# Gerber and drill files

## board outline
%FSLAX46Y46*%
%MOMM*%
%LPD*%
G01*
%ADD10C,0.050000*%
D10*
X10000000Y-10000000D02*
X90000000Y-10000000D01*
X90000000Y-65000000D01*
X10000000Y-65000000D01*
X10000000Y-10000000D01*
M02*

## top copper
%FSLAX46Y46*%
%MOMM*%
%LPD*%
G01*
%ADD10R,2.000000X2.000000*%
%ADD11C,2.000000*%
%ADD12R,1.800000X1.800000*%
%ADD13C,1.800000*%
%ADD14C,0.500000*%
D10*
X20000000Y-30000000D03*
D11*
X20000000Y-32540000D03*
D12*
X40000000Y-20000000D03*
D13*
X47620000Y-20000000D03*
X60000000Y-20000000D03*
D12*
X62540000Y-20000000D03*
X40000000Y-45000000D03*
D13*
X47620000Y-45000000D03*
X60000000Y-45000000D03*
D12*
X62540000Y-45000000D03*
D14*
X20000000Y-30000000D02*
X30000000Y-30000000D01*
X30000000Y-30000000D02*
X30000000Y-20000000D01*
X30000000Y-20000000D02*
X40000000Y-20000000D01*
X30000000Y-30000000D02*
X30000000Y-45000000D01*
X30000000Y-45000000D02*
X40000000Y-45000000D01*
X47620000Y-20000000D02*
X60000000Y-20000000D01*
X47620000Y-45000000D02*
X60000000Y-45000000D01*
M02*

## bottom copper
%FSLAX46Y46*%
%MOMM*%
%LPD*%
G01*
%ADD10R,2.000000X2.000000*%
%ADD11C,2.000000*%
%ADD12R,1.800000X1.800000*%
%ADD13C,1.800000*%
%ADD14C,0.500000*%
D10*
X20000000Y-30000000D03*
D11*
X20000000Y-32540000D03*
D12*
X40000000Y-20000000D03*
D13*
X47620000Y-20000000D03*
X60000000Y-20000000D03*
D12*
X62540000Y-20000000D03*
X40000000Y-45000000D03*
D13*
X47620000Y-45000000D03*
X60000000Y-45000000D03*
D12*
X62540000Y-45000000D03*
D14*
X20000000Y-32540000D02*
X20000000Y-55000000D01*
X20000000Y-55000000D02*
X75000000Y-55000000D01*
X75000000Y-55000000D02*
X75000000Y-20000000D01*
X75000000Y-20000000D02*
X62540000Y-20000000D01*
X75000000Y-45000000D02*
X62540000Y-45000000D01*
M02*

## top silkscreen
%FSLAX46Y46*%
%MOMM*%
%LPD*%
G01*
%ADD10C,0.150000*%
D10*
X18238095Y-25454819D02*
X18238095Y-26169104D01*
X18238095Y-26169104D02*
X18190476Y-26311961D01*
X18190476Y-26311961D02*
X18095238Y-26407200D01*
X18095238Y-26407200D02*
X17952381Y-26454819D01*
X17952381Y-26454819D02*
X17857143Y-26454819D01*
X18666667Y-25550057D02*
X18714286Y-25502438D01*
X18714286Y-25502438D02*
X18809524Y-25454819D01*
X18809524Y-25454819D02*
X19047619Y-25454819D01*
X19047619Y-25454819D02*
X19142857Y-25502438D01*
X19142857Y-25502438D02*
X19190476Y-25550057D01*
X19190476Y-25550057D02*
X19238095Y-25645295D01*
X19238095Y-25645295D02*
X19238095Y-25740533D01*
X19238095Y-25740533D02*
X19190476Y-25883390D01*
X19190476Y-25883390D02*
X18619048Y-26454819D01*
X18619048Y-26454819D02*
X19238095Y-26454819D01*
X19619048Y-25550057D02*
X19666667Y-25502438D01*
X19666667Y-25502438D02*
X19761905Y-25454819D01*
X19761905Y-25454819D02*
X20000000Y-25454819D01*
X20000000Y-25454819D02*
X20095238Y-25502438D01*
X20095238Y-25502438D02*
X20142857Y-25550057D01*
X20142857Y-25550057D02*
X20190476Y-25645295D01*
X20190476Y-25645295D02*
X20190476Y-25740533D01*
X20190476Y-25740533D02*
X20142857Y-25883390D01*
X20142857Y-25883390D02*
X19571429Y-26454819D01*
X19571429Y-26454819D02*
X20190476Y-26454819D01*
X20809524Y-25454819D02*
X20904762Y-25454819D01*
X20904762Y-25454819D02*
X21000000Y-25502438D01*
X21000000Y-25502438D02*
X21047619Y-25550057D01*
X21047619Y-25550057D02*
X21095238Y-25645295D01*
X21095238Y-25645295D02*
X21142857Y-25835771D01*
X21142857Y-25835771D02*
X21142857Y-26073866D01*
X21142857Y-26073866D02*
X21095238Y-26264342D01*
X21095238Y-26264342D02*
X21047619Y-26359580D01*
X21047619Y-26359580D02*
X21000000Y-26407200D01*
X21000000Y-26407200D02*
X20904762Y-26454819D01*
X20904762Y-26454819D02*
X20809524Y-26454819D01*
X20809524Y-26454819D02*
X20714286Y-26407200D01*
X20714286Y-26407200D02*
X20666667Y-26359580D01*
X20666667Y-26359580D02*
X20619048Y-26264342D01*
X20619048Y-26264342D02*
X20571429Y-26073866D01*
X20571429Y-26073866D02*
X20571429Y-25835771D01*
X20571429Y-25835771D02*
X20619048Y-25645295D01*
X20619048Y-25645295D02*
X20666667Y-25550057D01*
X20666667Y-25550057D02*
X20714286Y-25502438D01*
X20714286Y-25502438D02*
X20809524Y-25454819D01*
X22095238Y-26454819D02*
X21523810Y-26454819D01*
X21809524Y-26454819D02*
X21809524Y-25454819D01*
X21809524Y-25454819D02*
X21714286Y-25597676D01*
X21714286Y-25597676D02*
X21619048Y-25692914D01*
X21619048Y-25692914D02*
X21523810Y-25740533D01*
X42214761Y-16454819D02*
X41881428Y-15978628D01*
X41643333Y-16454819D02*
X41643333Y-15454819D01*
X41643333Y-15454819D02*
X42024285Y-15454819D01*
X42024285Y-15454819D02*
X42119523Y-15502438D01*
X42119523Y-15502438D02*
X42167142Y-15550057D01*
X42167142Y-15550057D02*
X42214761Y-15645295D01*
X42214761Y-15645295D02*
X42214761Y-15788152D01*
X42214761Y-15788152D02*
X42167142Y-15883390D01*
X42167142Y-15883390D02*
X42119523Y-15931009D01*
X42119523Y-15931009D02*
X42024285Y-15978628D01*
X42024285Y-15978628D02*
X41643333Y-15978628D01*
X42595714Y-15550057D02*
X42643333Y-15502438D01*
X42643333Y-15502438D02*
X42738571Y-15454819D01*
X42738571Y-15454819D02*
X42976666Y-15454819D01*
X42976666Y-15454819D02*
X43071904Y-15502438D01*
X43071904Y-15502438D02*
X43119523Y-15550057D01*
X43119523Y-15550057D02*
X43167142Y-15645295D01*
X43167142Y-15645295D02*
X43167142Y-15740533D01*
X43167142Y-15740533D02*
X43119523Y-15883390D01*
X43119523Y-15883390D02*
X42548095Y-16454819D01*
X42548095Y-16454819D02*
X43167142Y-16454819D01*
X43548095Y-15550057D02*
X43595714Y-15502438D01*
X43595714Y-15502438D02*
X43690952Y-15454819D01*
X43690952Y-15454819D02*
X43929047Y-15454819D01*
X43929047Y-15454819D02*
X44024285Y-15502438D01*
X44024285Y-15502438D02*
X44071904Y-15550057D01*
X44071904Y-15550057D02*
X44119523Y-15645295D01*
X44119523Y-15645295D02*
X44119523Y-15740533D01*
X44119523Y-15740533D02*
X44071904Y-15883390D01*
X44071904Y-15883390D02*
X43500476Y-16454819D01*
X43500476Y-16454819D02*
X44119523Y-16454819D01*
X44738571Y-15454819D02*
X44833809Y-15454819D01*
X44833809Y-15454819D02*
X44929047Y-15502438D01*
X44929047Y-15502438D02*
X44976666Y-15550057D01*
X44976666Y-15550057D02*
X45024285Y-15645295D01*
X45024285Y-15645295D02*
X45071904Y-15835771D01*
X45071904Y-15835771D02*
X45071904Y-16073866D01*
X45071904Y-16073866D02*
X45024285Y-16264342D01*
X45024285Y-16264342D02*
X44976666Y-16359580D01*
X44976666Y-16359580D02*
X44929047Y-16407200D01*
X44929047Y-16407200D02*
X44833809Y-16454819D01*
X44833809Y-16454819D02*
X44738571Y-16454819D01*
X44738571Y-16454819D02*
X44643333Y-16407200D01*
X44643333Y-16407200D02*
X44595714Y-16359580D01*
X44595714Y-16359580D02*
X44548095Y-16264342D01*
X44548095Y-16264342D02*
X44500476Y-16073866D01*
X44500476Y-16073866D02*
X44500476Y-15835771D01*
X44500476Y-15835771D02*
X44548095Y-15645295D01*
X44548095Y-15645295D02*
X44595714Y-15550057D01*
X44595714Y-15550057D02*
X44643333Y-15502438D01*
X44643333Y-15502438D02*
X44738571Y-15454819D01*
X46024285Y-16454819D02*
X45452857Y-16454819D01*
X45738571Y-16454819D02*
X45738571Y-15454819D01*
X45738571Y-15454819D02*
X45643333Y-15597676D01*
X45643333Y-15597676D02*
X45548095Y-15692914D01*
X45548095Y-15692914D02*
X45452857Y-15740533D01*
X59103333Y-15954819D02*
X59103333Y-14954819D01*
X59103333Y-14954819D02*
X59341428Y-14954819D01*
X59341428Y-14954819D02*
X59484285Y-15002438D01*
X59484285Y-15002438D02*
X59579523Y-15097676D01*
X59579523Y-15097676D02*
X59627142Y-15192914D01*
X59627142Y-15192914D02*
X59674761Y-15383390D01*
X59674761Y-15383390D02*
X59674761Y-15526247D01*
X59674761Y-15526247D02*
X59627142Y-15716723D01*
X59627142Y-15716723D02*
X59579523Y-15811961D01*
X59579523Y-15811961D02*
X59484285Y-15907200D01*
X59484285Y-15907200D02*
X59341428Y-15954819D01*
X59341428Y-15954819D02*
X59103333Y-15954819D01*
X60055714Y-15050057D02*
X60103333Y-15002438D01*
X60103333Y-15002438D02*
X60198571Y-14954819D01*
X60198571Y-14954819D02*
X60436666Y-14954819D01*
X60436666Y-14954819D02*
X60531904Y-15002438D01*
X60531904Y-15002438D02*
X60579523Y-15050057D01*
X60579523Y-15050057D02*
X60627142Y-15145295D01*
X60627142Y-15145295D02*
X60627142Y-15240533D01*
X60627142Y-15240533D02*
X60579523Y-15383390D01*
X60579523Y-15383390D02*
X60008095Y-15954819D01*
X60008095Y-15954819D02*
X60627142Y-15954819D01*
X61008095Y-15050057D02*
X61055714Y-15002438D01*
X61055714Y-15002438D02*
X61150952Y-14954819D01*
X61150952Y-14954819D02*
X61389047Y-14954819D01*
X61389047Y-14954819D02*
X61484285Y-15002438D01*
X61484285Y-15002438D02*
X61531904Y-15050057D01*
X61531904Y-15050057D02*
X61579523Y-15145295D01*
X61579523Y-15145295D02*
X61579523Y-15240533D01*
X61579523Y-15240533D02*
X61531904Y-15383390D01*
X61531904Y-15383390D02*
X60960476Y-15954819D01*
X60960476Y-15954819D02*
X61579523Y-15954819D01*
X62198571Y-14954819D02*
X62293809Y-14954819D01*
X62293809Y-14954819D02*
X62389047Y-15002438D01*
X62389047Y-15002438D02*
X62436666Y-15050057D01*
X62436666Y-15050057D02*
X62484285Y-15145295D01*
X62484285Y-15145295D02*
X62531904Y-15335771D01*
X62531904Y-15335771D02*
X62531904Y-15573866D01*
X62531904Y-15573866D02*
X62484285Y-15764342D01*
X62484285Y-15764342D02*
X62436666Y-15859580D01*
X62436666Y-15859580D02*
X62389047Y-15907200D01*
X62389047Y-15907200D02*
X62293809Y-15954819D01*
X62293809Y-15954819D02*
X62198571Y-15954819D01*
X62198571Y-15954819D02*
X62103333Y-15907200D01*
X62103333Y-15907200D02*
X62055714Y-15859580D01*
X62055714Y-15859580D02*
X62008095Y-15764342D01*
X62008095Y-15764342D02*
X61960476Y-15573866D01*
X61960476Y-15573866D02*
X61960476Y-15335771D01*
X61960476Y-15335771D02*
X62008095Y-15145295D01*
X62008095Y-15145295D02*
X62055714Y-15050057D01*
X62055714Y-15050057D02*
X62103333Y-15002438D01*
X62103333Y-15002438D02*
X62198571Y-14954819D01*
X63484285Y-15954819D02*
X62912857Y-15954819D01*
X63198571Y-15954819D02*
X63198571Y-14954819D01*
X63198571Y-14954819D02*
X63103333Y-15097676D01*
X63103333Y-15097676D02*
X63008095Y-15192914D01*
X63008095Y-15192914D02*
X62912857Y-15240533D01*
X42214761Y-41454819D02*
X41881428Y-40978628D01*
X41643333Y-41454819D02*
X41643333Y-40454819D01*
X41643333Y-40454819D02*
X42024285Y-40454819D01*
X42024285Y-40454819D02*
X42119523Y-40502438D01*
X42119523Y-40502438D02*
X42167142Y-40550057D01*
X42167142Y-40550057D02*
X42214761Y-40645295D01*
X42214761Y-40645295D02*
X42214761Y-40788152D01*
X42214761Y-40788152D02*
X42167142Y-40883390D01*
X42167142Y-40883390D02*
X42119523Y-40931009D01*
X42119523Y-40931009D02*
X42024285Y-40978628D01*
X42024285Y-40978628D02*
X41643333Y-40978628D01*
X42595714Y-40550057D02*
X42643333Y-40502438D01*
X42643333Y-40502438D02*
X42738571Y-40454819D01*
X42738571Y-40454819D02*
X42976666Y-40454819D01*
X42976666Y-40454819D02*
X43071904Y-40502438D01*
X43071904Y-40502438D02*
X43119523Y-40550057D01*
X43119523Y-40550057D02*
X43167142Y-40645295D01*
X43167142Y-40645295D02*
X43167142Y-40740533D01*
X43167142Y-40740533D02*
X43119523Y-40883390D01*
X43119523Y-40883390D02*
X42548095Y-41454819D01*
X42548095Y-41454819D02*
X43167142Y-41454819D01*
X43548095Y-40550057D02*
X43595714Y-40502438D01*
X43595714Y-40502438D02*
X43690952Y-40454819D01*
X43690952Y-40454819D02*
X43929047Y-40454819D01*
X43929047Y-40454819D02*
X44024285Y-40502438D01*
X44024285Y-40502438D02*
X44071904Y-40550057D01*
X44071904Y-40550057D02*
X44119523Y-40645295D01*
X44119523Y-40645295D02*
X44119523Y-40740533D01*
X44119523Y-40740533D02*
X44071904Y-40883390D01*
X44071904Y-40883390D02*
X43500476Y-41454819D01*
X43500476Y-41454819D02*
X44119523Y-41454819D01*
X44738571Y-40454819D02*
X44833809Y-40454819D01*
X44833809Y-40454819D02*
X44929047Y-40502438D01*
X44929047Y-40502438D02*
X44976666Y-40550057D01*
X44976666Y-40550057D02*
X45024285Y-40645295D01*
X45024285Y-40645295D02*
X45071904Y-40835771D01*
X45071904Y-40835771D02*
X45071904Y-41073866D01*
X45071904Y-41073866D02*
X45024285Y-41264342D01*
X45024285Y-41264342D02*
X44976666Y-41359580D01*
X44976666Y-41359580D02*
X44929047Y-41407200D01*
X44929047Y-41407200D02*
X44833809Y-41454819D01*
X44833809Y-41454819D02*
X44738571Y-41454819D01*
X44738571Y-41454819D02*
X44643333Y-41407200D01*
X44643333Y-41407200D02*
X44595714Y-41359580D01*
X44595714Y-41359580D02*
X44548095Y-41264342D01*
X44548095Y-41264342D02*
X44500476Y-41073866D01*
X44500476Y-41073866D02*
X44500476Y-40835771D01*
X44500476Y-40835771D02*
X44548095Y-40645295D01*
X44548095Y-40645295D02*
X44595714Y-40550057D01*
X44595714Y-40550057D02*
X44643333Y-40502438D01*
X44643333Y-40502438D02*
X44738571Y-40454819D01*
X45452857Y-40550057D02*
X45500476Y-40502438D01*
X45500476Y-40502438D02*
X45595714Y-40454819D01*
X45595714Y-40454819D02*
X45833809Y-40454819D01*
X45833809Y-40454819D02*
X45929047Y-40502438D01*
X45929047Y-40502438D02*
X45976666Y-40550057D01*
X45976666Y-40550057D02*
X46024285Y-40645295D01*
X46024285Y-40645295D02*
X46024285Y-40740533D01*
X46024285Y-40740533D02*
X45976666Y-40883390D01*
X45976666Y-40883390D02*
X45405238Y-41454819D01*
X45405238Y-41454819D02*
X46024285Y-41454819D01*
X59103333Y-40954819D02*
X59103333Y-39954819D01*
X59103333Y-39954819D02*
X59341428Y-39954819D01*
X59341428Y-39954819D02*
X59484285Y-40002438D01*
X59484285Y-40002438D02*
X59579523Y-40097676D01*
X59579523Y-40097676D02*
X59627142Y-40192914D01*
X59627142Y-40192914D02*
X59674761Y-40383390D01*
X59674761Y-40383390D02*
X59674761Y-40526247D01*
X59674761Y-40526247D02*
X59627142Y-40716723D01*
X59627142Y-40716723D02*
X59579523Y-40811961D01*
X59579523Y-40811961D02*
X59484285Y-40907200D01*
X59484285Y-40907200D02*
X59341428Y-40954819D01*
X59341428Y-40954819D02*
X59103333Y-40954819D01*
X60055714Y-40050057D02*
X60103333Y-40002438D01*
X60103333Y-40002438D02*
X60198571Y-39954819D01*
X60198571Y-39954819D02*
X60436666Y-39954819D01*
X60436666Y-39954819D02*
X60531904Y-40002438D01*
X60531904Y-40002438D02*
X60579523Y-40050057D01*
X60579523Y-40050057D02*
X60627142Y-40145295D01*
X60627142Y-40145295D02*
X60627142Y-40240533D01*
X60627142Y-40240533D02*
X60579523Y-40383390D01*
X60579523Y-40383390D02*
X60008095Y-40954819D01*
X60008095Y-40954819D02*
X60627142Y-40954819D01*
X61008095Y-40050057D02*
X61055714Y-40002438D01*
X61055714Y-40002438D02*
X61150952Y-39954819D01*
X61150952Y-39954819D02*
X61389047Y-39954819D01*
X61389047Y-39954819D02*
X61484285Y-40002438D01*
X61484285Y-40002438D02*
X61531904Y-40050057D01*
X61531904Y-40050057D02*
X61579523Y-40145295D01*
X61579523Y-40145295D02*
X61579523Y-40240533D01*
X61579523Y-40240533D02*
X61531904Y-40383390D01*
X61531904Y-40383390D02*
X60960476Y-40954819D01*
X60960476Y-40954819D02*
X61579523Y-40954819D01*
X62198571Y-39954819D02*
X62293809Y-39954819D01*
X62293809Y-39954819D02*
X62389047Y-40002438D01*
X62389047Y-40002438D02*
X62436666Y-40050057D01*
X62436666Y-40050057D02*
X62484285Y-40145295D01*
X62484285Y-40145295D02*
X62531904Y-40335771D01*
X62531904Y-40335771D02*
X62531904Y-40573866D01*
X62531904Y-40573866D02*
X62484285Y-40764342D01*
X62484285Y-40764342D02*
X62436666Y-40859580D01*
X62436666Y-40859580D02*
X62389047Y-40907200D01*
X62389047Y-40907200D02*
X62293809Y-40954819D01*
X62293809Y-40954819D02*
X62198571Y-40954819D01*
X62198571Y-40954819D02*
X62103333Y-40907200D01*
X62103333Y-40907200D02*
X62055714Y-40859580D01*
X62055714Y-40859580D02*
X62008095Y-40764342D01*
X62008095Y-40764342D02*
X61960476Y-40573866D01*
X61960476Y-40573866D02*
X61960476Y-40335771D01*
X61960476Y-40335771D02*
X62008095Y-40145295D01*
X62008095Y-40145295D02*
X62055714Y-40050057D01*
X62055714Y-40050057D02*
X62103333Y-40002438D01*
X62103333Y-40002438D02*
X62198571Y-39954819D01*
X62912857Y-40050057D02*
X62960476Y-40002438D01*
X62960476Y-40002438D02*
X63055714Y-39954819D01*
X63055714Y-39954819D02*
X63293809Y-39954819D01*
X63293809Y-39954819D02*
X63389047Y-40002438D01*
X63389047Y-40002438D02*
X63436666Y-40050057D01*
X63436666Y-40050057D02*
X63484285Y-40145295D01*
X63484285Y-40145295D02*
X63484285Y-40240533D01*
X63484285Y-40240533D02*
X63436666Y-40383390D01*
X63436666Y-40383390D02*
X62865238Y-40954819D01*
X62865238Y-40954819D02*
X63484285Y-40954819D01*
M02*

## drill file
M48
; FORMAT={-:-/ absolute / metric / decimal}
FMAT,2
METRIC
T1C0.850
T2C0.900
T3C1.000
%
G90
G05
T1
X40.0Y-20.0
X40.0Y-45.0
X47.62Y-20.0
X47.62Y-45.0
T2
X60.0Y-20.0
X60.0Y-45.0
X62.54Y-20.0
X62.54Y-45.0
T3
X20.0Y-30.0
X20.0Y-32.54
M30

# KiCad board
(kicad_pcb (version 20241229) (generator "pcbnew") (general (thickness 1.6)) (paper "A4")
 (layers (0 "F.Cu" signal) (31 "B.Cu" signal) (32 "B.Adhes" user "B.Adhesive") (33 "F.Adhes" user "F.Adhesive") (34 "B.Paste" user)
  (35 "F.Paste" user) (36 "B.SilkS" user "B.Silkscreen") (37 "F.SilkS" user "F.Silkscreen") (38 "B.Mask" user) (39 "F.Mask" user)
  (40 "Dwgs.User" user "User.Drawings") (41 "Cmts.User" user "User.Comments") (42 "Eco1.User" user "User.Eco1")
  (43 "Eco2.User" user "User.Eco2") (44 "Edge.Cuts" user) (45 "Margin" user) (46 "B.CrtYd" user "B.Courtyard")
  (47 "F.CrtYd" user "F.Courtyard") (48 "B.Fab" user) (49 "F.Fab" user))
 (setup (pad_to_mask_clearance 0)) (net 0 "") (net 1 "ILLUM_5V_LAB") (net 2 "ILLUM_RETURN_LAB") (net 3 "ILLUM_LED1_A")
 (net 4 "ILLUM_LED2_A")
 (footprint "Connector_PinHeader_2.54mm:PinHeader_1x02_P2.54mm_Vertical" (layer "F.Cu") (at 20 30)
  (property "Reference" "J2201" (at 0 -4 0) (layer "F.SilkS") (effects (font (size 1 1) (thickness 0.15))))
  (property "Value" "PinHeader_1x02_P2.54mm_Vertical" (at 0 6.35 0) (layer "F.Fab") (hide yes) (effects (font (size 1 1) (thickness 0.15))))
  (pad "1" thru_hole rect (at 0 0) (size 2 2) (drill 1) (layers "*.Cu" "*.Mask") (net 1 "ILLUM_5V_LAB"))
  (pad "2" thru_hole circle (at 0 2.54) (size 2 2) (drill 1) (layers "*.Cu" "*.Mask") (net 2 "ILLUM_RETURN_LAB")))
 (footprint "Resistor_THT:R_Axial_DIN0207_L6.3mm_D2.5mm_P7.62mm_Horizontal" (layer "F.Cu") (at 40 20)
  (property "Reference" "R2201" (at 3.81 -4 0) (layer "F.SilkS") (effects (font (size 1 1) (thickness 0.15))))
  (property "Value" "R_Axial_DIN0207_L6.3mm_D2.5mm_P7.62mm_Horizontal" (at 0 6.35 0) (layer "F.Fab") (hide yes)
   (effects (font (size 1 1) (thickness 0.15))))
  (pad "1" thru_hole rect (at 0 0) (size 1.8 1.8) (drill 0.85) (layers "*.Cu" "*.Mask") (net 1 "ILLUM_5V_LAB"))
  (pad "2" thru_hole circle (at 7.62 0) (size 1.8 1.8) (drill 0.85) (layers "*.Cu" "*.Mask") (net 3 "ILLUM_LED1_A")))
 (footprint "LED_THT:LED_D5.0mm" (layer "F.Cu") (at 60 20)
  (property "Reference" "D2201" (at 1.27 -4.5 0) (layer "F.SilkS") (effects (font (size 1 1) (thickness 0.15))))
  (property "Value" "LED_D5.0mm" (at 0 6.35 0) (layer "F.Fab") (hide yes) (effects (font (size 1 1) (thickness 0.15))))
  (pad "2" thru_hole circle (at 0 0) (size 1.8 1.8) (drill 0.9) (layers "*.Cu" "*.Mask") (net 3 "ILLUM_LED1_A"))
  (pad "1" thru_hole rect (at 2.54 0) (size 1.8 1.8) (drill 0.9) (layers "*.Cu" "*.Mask") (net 2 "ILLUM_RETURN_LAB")))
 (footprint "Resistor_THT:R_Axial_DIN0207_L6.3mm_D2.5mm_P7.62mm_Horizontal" (layer "F.Cu") (at 40 45)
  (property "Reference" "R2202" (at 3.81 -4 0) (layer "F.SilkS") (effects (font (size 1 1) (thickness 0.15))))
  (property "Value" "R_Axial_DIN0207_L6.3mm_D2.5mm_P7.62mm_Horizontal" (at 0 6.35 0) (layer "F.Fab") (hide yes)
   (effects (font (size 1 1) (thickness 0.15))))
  (pad "1" thru_hole rect (at 0 0) (size 1.8 1.8) (drill 0.85) (layers "*.Cu" "*.Mask") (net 1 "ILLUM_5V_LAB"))
  (pad "2" thru_hole circle (at 7.62 0) (size 1.8 1.8) (drill 0.85) (layers "*.Cu" "*.Mask") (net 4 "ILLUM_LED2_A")))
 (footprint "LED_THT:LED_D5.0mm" (layer "F.Cu") (at 60 45)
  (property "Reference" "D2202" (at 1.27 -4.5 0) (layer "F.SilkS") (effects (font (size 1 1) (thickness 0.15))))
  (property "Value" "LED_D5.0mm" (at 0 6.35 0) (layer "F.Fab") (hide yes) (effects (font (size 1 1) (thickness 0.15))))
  (pad "2" thru_hole circle (at 0 0) (size 1.8 1.8) (drill 0.9) (layers "*.Cu" "*.Mask") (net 4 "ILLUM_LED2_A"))
  (pad "1" thru_hole rect (at 2.54 0) (size 1.8 1.8) (drill 0.9) (layers "*.Cu" "*.Mask") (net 2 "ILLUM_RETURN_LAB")))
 (segment (start 20 30) (end 30 30) (width 0.5) (layer "F.Cu") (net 1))
 (segment (start 30 30) (end 30 20) (width 0.5) (layer "F.Cu") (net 1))
 (segment (start 30 20) (end 40 20) (width 0.5) (layer "F.Cu") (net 1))
 (segment (start 30 30) (end 30 45) (width 0.5) (layer "F.Cu") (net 1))
 (segment (start 30 45) (end 40 45) (width 0.5) (layer "F.Cu") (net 1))
 (segment (start 47.62 20) (end 60 20) (width 0.5) (layer "F.Cu") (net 3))
 (segment (start 47.62 45) (end 60 45) (width 0.5) (layer "F.Cu") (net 4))
 (segment (start 20 32.54) (end 20 55) (width 0.5) (layer "B.Cu") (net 2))
 (segment (start 20 55) (end 75 55) (width 0.5) (layer "B.Cu") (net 2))
 (segment (start 75 55) (end 75 20) (width 0.5) (layer "B.Cu") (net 2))
 (segment (start 75 20) (end 62.54 20) (width 0.5) (layer "B.Cu") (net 2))
 (segment (start 75 45) (end 62.54 45) (width 0.5) (layer "B.Cu") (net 2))
 (gr_rect (start 10 10) (end 90 65) (stroke (width 0.05) (type default)) (fill none) (layer "Edge.Cuts")))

